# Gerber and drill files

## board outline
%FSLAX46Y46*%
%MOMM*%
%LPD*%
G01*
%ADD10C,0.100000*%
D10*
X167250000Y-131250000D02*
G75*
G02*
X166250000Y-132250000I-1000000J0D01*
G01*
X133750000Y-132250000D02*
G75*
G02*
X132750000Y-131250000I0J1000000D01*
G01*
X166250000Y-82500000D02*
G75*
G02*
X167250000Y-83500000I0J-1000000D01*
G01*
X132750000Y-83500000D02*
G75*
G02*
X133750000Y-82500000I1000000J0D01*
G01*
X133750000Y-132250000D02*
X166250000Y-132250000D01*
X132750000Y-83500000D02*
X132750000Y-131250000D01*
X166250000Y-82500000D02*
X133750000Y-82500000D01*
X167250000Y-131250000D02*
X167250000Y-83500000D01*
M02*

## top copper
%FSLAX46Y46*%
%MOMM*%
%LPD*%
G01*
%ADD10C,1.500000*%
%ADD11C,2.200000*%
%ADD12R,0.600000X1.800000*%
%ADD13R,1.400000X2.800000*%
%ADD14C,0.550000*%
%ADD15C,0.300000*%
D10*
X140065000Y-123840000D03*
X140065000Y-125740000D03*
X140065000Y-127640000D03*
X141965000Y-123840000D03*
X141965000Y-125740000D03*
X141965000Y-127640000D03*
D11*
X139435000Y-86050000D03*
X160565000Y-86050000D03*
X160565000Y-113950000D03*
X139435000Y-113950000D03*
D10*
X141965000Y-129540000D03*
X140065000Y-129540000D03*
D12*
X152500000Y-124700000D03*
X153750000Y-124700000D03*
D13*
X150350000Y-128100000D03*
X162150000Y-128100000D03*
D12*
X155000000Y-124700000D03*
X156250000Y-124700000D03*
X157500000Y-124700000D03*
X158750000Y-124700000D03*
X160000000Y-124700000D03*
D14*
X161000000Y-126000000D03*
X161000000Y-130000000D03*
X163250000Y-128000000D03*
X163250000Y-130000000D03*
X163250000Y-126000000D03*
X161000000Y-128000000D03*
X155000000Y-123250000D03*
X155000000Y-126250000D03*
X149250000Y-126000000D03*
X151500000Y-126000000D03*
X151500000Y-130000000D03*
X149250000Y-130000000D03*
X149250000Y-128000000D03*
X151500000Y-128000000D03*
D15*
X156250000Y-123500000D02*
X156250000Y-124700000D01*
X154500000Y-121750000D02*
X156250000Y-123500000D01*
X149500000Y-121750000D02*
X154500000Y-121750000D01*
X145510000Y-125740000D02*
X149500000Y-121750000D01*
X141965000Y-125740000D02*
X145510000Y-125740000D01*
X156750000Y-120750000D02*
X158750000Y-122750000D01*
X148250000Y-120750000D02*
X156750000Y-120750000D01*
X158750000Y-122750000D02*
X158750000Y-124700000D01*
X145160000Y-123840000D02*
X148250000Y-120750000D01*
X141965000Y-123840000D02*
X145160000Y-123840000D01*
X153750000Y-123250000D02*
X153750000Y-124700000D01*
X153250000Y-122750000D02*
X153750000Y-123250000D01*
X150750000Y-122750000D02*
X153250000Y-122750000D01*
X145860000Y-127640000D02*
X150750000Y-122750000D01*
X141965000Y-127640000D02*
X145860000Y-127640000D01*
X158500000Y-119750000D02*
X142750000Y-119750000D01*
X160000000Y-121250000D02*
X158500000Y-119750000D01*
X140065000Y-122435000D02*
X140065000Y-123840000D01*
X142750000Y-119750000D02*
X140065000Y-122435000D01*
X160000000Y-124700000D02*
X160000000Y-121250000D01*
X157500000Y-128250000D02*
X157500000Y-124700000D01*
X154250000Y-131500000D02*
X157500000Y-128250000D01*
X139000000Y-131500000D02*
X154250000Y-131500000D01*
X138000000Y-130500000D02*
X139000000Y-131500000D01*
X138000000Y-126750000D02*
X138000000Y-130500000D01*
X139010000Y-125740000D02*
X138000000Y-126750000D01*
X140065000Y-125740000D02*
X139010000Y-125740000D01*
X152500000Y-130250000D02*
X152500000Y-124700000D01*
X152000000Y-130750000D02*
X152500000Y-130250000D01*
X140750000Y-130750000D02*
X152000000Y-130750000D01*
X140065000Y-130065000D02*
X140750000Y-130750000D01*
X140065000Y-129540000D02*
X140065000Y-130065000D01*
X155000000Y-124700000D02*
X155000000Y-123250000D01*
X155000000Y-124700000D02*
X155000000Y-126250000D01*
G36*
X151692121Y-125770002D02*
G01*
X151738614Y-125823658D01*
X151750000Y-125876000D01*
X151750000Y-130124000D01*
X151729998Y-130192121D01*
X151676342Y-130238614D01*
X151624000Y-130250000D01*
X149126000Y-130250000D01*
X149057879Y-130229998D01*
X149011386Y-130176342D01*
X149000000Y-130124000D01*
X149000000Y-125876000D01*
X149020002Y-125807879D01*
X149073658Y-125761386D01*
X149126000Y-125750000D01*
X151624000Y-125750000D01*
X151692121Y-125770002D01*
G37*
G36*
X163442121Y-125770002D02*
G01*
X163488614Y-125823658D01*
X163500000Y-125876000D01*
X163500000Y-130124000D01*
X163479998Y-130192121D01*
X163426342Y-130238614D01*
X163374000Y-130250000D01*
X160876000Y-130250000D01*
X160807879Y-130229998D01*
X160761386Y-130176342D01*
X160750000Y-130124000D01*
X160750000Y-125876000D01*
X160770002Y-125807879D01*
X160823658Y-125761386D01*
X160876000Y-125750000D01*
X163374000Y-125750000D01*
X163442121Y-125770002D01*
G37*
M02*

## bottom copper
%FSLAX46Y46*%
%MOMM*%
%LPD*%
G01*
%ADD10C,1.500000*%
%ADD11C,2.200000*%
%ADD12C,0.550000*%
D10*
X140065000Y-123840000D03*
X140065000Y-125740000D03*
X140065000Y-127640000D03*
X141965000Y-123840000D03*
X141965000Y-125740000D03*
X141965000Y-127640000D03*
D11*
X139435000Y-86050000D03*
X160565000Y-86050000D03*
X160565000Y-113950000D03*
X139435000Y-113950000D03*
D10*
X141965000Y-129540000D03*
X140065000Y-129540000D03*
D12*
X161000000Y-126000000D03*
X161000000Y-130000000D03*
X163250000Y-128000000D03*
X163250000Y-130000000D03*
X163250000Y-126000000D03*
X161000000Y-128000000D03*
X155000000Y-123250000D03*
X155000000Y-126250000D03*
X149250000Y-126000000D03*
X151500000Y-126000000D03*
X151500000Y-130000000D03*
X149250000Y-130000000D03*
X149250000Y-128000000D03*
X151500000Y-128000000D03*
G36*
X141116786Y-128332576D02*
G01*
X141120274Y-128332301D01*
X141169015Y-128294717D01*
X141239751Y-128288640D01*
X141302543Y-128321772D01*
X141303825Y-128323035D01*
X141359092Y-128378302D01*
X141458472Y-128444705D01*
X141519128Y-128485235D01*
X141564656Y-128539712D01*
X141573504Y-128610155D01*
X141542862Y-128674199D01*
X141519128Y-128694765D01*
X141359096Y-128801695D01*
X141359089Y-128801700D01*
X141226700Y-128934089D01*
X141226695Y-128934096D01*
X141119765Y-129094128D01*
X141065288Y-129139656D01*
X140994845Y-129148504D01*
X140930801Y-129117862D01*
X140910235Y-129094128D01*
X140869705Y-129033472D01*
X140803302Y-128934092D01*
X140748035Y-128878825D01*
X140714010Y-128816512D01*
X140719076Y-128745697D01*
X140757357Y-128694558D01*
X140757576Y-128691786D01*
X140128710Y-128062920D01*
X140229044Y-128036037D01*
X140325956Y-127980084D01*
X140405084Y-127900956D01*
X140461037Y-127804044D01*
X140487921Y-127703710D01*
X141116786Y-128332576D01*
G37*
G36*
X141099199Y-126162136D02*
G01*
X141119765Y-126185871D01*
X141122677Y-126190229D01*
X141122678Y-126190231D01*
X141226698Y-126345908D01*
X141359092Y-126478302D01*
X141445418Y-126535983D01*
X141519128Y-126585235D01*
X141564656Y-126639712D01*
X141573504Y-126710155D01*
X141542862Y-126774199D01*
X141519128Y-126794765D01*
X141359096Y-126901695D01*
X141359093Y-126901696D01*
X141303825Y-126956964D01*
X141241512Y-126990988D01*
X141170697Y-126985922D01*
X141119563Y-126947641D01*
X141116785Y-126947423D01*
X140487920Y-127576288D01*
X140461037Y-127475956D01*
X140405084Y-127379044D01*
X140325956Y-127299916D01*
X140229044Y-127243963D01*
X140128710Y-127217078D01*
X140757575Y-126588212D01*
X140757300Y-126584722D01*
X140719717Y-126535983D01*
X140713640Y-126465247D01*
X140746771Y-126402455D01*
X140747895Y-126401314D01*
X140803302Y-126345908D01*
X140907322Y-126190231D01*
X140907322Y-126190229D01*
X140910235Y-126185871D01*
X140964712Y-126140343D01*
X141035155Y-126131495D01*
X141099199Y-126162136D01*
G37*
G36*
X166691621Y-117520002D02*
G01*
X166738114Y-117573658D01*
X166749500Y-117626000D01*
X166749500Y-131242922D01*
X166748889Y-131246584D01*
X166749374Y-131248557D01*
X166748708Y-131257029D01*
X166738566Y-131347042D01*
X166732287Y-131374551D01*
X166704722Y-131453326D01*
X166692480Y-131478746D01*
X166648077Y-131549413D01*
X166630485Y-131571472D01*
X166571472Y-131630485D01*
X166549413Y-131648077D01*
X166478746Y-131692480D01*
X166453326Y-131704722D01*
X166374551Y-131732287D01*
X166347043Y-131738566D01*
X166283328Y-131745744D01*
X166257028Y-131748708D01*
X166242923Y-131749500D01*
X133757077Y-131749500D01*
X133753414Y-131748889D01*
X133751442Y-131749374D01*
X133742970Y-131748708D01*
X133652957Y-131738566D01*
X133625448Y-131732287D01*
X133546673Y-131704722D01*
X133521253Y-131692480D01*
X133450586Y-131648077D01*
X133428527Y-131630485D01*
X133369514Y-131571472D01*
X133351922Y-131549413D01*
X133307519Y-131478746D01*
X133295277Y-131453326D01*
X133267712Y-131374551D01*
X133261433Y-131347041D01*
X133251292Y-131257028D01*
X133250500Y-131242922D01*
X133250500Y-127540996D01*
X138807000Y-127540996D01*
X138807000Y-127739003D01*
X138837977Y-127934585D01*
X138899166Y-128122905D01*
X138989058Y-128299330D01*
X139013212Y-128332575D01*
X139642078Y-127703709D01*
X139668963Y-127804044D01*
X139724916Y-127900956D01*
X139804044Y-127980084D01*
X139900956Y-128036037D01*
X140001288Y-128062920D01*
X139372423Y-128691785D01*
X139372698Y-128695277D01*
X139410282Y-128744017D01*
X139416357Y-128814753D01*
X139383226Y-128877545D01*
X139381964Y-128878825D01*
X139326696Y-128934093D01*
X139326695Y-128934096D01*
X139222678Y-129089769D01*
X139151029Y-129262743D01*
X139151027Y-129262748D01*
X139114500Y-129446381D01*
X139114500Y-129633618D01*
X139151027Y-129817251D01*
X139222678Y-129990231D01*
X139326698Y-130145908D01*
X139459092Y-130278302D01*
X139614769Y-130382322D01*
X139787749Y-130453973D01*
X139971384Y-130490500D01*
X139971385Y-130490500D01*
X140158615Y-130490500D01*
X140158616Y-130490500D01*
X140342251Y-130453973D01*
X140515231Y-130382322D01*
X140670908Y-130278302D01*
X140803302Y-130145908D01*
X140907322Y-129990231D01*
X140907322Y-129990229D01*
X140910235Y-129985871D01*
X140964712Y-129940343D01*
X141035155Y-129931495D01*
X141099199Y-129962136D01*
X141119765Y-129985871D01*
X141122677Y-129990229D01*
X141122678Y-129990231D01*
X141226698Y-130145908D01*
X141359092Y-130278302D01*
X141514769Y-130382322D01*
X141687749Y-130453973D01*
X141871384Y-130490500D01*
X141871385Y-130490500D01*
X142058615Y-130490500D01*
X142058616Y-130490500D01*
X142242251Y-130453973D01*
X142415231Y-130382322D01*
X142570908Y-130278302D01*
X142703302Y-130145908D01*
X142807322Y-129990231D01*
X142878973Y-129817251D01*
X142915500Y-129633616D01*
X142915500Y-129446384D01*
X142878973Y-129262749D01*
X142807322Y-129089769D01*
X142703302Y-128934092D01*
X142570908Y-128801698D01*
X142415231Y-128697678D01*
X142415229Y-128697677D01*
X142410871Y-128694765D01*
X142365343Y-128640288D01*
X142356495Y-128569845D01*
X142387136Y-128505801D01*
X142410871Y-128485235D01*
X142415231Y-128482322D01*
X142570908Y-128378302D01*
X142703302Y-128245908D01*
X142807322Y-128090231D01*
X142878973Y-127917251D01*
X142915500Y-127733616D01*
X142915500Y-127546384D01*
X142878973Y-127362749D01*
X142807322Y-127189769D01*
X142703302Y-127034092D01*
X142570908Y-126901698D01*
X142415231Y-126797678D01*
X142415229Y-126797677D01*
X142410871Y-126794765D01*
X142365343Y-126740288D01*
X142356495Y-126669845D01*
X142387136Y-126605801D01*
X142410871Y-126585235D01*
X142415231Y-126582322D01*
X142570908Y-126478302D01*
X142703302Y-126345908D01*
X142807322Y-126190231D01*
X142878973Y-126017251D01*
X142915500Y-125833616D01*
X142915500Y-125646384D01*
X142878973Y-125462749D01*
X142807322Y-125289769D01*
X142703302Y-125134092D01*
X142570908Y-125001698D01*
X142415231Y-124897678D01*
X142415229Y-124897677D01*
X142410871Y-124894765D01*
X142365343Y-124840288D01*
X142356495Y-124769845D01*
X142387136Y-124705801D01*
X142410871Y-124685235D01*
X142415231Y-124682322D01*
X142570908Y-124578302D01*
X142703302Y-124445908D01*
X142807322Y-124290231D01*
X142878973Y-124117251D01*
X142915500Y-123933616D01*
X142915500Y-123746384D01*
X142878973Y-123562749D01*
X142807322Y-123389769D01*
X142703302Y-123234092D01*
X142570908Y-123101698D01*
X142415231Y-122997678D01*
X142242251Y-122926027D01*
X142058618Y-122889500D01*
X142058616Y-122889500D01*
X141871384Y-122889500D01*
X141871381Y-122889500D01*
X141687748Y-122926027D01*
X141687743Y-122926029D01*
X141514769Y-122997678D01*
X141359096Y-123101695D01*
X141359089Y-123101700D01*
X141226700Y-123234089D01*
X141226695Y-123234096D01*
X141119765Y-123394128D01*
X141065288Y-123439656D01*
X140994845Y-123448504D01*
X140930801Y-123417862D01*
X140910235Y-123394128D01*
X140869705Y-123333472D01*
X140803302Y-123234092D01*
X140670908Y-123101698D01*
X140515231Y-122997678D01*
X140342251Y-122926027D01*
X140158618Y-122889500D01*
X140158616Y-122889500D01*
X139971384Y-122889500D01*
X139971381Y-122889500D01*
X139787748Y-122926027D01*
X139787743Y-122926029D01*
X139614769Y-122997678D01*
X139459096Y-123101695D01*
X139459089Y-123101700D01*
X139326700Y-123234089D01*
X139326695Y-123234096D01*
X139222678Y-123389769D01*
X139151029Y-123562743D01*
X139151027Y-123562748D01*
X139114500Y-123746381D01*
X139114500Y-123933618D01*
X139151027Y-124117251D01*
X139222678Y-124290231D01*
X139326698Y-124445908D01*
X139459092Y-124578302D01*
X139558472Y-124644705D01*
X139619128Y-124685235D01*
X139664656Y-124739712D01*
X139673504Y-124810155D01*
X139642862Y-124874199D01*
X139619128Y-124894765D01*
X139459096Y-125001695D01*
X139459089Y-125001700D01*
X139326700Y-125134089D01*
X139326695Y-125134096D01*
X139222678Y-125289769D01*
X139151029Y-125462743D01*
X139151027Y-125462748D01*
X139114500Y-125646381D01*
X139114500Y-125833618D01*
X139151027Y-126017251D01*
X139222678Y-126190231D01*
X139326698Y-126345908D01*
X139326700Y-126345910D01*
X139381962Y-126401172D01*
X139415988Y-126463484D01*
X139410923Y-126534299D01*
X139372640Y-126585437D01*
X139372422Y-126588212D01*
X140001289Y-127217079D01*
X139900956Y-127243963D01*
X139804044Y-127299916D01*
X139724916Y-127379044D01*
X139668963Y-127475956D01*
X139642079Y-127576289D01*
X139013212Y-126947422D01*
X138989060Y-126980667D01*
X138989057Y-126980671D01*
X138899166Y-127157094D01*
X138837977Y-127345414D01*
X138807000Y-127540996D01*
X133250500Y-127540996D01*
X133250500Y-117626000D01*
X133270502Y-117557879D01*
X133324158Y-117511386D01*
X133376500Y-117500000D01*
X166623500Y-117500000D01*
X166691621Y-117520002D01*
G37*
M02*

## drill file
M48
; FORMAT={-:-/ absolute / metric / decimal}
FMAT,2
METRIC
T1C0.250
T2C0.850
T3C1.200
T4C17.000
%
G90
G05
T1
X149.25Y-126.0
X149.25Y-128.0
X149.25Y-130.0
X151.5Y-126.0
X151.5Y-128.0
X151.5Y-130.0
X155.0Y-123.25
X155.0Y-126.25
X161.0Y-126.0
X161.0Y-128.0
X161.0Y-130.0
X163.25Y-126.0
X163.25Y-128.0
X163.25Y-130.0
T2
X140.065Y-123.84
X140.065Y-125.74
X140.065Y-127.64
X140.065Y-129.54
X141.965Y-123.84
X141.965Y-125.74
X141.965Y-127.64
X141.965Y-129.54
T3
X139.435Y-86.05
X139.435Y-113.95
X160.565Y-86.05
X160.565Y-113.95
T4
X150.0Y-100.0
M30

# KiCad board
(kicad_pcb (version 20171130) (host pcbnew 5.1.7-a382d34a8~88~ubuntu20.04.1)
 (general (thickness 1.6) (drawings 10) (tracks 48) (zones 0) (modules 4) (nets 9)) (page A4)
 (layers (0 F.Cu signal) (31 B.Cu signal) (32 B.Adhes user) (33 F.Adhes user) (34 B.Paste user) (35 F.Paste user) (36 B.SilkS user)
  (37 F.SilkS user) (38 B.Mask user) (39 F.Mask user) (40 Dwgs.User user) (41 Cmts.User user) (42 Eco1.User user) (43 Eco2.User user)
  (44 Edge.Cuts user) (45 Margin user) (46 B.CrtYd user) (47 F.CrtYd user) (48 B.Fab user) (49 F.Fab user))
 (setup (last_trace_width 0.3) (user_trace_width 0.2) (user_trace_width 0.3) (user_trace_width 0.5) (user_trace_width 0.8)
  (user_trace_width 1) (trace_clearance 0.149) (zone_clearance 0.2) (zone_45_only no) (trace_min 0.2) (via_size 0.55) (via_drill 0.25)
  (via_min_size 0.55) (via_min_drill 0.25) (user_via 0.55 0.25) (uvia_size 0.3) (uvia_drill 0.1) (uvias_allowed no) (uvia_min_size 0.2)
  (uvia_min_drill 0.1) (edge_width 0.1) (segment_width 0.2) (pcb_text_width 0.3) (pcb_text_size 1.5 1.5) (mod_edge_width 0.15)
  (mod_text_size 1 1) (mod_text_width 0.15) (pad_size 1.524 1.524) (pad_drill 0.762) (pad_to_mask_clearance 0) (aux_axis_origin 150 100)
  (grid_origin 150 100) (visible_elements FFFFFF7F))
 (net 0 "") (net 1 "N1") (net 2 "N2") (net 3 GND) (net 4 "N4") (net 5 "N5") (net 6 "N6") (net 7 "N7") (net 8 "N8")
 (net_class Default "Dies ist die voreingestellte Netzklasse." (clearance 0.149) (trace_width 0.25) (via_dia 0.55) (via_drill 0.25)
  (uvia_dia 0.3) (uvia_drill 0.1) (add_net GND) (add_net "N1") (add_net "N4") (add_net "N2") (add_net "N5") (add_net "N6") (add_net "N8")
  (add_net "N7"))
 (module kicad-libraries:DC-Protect (layer B.Cu) (at 150 100 180)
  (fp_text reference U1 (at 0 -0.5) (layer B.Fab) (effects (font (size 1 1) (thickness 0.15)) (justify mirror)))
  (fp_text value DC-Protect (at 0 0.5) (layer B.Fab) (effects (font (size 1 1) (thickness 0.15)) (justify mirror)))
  (pad 1 thru_hole circle (at 9.935 -23.84 180) (size 1.5 1.5) (drill 0.85) (layers *.Cu *.Mask) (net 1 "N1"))
  (pad 3 thru_hole circle (at 9.935 -25.74 180) (size 1.5 1.5) (drill 0.85) (layers *.Cu *.Mask) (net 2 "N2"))
  (pad 5 thru_hole circle (at 9.935 -27.64 180) (size 1.5 1.5) (drill 0.85) (layers *.Cu *.Mask) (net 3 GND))
  (pad 2 thru_hole circle (at 8.035 -23.84 180) (size 1.5 1.5) (drill 0.85) (layers *.Cu *.Mask) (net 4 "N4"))
  (pad 4 thru_hole circle (at 8.035 -25.74 180) (size 1.5 1.5) (drill 0.85) (layers *.Cu *.Mask) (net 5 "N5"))
  (pad 6 thru_hole circle (at 8.035 -27.64 180) (size 1.5 1.5) (drill 0.85) (layers *.Cu *.Mask) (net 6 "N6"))
  (pad "" np_thru_hole circle (at 0 0 180) (size 17 17) (drill 17) (layers *.Cu *.Mask))
  (pad "" thru_hole circle (at 10.565 13.95 180) (size 2.2 2.2) (drill 1.2) (layers *.Cu *.Mask))
  (pad "" thru_hole circle (at -10.565 13.95 180) (size 2.2 2.2) (drill 1.2) (layers *.Cu *.Mask))
  (pad "" thru_hole circle (at -10.565 -13.95 180) (size 2.2 2.2) (drill 1.2) (layers *.Cu *.Mask))
  (pad "" thru_hole circle (at 10.565 -13.95 180) (size 2.2 2.2) (drill 1.2) (layers *.Cu *.Mask))
  (pad 8 thru_hole circle (at 8.035 -29.54 180) (size 1.5 1.5) (drill 0.85) (layers *.Cu *.Mask) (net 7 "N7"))
  (pad 7 thru_hole circle (at 9.935 -29.54 180) (size 1.5 1.5) (drill 0.85) (layers *.Cu *.Mask) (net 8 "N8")))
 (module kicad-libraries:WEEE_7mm (layer F.Cu) (at 150 87.1 180)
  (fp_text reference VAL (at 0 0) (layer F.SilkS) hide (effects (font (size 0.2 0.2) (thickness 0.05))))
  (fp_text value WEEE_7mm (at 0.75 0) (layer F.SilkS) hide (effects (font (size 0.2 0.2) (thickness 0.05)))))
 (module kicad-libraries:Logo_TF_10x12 (layer F.Cu) (at 149.96 114.89 180)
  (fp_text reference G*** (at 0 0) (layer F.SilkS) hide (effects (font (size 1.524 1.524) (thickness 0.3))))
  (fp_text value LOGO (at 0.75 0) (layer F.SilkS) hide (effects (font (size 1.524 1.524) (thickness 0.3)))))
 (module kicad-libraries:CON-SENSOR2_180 (layer F.Cu) (at 156.25 129.5)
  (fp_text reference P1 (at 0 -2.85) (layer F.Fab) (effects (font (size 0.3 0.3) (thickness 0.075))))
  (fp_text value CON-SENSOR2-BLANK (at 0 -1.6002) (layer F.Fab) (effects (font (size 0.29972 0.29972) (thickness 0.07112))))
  (pad 7 smd rect (at -3.75 -4.8) (size 0.6 1.8) (layers F.Cu F.Paste F.Mask) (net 8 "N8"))
  (pad 6 smd rect (at -2.5 -4.8) (size 0.6 1.8) (layers F.Cu F.Paste F.Mask) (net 6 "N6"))
  (pad EP smd rect (at -5.9 -1.4) (size 1.4 2.8) (layers F.Cu F.Paste F.Mask) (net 3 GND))
  (pad EP smd rect (at 5.9 -1.4) (size 1.4 2.8) (layers F.Cu F.Paste F.Mask) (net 3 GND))
  (pad 5 smd rect (at -1.25 -4.8) (size 0.6 1.8) (layers F.Cu F.Paste F.Mask) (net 3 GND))
  (pad 4 smd rect (at 0 -4.8) (size 0.6 1.8) (layers F.Cu F.Paste F.Mask) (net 5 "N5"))
  (pad 3 smd rect (at 1.25 -4.8) (size 0.6 1.8) (layers F.Cu F.Paste F.Mask) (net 2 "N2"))
  (pad 2 smd rect (at 2.5 -4.8) (size 0.6 1.8) (layers F.Cu F.Paste F.Mask) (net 4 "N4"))
  (pad 1 smd rect (at 3.75 -4.8) (size 0.6 1.8) (layers F.Cu F.Paste F.Mask) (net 1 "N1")))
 (gr_arc (start 166.25 131.25) (end 166.25 132.25) (angle -90) (layer Edge.Cuts) (width 0.1))
 (gr_arc (start 133.75 131.25) (end 132.75 131.25) (angle -90) (layer Edge.Cuts) (width 0.1))
 (gr_arc (start 166.25 83.5) (end 167.25 83.5) (angle -90) (layer Edge.Cuts) (width 0.1))
 (gr_arc (start 133.75 83.5) (end 133.75 82.5) (angle -90) (layer Edge.Cuts) (width 0.1))
 (gr_line (start 133.75 132.25) (end 166.25 132.25) (layer Edge.Cuts) (width 0.1))
 (gr_line (start 132.75 83.5) (end 132.75 131.25) (layer Edge.Cuts) (width 0.1))
 (gr_line (start 166.25 82.5) (end 133.75 82.5) (layer Edge.Cuts) (width 0.1))
 (gr_line (start 167.25 131.25) (end 167.25 83.5) (layer Edge.Cuts) (width 0.1))
 (via (at 161 126) (size 0.55) (drill 0.25) (layers F.Cu B.Cu) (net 3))
 (via (at 161 130) (size 0.55) (drill 0.25) (layers F.Cu B.Cu) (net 3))
 (via (at 163.25 128) (size 0.55) (drill 0.25) (layers F.Cu B.Cu) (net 3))
 (via (at 163.25 130) (size 0.55) (drill 0.25) (layers F.Cu B.Cu) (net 3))
 (via (at 163.25 126) (size 0.55) (drill 0.25) (layers F.Cu B.Cu) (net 3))
 (via (at 161 128) (size 0.55) (drill 0.25) (layers F.Cu B.Cu) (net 3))
 (segment (start 156.25 123.5) (end 156.25 124.7) (width 0.3) (layer F.Cu) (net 5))
 (segment (start 154.5 121.75) (end 156.25 123.5) (width 0.3) (layer F.Cu) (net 5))
 (segment (start 149.5 121.75) (end 154.5 121.75) (width 0.3) (layer F.Cu) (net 5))
 (segment (start 145.51 125.74) (end 149.5 121.75) (width 0.3) (layer F.Cu) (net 5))
 (segment (start 141.965 125.74) (end 145.51 125.74) (width 0.3) (layer F.Cu) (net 5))
 (segment (start 156.75 120.75) (end 158.75 122.75) (width 0.3) (layer F.Cu) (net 4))
 (segment (start 148.25 120.75) (end 156.75 120.75) (width 0.3) (layer F.Cu) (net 4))
 (segment (start 158.75 122.75) (end 158.75 124.7) (width 0.3) (layer F.Cu) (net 4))
 (segment (start 145.16 123.84) (end 148.25 120.75) (width 0.3) (layer F.Cu) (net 4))
 (segment (start 141.965 123.84) (end 145.16 123.84) (width 0.3) (layer F.Cu) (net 4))
 (segment (start 153.75 123.25) (end 153.75 124.7) (width 0.3) (layer F.Cu) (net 6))
 (segment (start 153.25 122.75) (end 153.75 123.25) (width 0.3) (layer F.Cu) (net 6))
 (segment (start 150.75 122.75) (end 153.25 122.75) (width 0.3) (layer F.Cu) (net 6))
 (segment (start 145.86 127.64) (end 150.75 122.75) (width 0.3) (layer F.Cu) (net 6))
 (segment (start 141.965 127.64) (end 145.86 127.64) (width 0.3) (layer F.Cu) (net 6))
 (segment (start 158.5 119.75) (end 142.75 119.75) (width 0.3) (layer F.Cu) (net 1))
 (segment (start 160 121.25) (end 158.5 119.75) (width 0.3) (layer F.Cu) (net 1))
 (segment (start 140.065 122.435) (end 140.065 123.84) (width 0.3) (layer F.Cu) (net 1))
 (segment (start 142.75 119.75) (end 140.065 122.435) (width 0.3) (layer F.Cu) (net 1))
 (segment (start 160 124.7) (end 160 121.25) (width 0.3) (layer F.Cu) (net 1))
 (segment (start 157.5 128.25) (end 157.5 124.7) (width 0.3) (layer F.Cu) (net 2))
 (segment (start 154.25 131.5) (end 157.5 128.25) (width 0.3) (layer F.Cu) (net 2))
 (segment (start 139 131.5) (end 154.25 131.5) (width 0.3) (layer F.Cu) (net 2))
 (segment (start 138 130.5) (end 139 131.5) (width 0.3) (layer F.Cu) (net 2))
 (segment (start 138 126.75) (end 138 130.5) (width 0.3) (layer F.Cu) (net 2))
 (segment (start 139.01 125.74) (end 138 126.75) (width 0.3) (layer F.Cu) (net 2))
 (segment (start 140.065 125.74) (end 139.01 125.74) (width 0.3) (layer F.Cu) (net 2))
 (segment (start 152.5 130.25) (end 152.5 124.7) (width 0.3) (layer F.Cu) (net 8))
 (segment (start 152 130.75) (end 152.5 130.25) (width 0.3) (layer F.Cu) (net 8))
 (segment (start 140.75 130.75) (end 152 130.75) (width 0.3) (layer F.Cu) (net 8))
 (segment (start 140.065 130.065) (end 140.75 130.75) (width 0.3) (layer F.Cu) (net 8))
 (segment (start 140.065 129.54) (end 140.065 130.065) (width 0.3) (layer F.Cu) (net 8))
 (via (at 155 123.25) (size 0.55) (drill 0.25) (layers F.Cu B.Cu) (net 3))
 (segment (start 155 124.7) (end 155 123.25) (width 0.3) (layer F.Cu) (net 3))
 (via (at 155 126.25) (size 0.55) (drill 0.25) (layers F.Cu B.Cu) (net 3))
 (segment (start 155 124.7) (end 155 126.25) (width 0.3) (layer F.Cu) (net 3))
 (via (at 149.25 126) (size 0.55) (drill 0.25) (layers F.Cu B.Cu) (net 3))
 (via (at 151.5 126) (size 0.55) (drill 0.25) (layers F.Cu B.Cu) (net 3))
 (via (at 151.5 130) (size 0.55) (drill 0.25) (layers F.Cu B.Cu) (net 3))
 (via (at 149.25 130) (size 0.55) (drill 0.25) (layers F.Cu B.Cu) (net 3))
 (via (at 149.25 128) (size 0.55) (drill 0.25) (layers F.Cu B.Cu) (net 3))
 (via (at 151.5 128) (size 0.55) (drill 0.25) (layers F.Cu B.Cu) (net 3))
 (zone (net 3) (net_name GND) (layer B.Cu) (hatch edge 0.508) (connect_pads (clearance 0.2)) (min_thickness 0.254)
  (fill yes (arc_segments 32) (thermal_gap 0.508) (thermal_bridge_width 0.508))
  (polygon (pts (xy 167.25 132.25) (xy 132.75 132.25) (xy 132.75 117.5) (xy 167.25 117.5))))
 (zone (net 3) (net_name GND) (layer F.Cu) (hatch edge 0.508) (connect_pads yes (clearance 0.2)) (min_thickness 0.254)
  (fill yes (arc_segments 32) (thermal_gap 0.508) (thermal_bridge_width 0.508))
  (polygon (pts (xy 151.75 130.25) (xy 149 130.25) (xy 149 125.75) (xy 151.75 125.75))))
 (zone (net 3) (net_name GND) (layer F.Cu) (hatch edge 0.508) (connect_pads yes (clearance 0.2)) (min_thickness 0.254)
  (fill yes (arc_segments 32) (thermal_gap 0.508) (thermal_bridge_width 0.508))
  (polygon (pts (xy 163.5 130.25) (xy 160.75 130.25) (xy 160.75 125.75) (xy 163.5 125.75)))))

